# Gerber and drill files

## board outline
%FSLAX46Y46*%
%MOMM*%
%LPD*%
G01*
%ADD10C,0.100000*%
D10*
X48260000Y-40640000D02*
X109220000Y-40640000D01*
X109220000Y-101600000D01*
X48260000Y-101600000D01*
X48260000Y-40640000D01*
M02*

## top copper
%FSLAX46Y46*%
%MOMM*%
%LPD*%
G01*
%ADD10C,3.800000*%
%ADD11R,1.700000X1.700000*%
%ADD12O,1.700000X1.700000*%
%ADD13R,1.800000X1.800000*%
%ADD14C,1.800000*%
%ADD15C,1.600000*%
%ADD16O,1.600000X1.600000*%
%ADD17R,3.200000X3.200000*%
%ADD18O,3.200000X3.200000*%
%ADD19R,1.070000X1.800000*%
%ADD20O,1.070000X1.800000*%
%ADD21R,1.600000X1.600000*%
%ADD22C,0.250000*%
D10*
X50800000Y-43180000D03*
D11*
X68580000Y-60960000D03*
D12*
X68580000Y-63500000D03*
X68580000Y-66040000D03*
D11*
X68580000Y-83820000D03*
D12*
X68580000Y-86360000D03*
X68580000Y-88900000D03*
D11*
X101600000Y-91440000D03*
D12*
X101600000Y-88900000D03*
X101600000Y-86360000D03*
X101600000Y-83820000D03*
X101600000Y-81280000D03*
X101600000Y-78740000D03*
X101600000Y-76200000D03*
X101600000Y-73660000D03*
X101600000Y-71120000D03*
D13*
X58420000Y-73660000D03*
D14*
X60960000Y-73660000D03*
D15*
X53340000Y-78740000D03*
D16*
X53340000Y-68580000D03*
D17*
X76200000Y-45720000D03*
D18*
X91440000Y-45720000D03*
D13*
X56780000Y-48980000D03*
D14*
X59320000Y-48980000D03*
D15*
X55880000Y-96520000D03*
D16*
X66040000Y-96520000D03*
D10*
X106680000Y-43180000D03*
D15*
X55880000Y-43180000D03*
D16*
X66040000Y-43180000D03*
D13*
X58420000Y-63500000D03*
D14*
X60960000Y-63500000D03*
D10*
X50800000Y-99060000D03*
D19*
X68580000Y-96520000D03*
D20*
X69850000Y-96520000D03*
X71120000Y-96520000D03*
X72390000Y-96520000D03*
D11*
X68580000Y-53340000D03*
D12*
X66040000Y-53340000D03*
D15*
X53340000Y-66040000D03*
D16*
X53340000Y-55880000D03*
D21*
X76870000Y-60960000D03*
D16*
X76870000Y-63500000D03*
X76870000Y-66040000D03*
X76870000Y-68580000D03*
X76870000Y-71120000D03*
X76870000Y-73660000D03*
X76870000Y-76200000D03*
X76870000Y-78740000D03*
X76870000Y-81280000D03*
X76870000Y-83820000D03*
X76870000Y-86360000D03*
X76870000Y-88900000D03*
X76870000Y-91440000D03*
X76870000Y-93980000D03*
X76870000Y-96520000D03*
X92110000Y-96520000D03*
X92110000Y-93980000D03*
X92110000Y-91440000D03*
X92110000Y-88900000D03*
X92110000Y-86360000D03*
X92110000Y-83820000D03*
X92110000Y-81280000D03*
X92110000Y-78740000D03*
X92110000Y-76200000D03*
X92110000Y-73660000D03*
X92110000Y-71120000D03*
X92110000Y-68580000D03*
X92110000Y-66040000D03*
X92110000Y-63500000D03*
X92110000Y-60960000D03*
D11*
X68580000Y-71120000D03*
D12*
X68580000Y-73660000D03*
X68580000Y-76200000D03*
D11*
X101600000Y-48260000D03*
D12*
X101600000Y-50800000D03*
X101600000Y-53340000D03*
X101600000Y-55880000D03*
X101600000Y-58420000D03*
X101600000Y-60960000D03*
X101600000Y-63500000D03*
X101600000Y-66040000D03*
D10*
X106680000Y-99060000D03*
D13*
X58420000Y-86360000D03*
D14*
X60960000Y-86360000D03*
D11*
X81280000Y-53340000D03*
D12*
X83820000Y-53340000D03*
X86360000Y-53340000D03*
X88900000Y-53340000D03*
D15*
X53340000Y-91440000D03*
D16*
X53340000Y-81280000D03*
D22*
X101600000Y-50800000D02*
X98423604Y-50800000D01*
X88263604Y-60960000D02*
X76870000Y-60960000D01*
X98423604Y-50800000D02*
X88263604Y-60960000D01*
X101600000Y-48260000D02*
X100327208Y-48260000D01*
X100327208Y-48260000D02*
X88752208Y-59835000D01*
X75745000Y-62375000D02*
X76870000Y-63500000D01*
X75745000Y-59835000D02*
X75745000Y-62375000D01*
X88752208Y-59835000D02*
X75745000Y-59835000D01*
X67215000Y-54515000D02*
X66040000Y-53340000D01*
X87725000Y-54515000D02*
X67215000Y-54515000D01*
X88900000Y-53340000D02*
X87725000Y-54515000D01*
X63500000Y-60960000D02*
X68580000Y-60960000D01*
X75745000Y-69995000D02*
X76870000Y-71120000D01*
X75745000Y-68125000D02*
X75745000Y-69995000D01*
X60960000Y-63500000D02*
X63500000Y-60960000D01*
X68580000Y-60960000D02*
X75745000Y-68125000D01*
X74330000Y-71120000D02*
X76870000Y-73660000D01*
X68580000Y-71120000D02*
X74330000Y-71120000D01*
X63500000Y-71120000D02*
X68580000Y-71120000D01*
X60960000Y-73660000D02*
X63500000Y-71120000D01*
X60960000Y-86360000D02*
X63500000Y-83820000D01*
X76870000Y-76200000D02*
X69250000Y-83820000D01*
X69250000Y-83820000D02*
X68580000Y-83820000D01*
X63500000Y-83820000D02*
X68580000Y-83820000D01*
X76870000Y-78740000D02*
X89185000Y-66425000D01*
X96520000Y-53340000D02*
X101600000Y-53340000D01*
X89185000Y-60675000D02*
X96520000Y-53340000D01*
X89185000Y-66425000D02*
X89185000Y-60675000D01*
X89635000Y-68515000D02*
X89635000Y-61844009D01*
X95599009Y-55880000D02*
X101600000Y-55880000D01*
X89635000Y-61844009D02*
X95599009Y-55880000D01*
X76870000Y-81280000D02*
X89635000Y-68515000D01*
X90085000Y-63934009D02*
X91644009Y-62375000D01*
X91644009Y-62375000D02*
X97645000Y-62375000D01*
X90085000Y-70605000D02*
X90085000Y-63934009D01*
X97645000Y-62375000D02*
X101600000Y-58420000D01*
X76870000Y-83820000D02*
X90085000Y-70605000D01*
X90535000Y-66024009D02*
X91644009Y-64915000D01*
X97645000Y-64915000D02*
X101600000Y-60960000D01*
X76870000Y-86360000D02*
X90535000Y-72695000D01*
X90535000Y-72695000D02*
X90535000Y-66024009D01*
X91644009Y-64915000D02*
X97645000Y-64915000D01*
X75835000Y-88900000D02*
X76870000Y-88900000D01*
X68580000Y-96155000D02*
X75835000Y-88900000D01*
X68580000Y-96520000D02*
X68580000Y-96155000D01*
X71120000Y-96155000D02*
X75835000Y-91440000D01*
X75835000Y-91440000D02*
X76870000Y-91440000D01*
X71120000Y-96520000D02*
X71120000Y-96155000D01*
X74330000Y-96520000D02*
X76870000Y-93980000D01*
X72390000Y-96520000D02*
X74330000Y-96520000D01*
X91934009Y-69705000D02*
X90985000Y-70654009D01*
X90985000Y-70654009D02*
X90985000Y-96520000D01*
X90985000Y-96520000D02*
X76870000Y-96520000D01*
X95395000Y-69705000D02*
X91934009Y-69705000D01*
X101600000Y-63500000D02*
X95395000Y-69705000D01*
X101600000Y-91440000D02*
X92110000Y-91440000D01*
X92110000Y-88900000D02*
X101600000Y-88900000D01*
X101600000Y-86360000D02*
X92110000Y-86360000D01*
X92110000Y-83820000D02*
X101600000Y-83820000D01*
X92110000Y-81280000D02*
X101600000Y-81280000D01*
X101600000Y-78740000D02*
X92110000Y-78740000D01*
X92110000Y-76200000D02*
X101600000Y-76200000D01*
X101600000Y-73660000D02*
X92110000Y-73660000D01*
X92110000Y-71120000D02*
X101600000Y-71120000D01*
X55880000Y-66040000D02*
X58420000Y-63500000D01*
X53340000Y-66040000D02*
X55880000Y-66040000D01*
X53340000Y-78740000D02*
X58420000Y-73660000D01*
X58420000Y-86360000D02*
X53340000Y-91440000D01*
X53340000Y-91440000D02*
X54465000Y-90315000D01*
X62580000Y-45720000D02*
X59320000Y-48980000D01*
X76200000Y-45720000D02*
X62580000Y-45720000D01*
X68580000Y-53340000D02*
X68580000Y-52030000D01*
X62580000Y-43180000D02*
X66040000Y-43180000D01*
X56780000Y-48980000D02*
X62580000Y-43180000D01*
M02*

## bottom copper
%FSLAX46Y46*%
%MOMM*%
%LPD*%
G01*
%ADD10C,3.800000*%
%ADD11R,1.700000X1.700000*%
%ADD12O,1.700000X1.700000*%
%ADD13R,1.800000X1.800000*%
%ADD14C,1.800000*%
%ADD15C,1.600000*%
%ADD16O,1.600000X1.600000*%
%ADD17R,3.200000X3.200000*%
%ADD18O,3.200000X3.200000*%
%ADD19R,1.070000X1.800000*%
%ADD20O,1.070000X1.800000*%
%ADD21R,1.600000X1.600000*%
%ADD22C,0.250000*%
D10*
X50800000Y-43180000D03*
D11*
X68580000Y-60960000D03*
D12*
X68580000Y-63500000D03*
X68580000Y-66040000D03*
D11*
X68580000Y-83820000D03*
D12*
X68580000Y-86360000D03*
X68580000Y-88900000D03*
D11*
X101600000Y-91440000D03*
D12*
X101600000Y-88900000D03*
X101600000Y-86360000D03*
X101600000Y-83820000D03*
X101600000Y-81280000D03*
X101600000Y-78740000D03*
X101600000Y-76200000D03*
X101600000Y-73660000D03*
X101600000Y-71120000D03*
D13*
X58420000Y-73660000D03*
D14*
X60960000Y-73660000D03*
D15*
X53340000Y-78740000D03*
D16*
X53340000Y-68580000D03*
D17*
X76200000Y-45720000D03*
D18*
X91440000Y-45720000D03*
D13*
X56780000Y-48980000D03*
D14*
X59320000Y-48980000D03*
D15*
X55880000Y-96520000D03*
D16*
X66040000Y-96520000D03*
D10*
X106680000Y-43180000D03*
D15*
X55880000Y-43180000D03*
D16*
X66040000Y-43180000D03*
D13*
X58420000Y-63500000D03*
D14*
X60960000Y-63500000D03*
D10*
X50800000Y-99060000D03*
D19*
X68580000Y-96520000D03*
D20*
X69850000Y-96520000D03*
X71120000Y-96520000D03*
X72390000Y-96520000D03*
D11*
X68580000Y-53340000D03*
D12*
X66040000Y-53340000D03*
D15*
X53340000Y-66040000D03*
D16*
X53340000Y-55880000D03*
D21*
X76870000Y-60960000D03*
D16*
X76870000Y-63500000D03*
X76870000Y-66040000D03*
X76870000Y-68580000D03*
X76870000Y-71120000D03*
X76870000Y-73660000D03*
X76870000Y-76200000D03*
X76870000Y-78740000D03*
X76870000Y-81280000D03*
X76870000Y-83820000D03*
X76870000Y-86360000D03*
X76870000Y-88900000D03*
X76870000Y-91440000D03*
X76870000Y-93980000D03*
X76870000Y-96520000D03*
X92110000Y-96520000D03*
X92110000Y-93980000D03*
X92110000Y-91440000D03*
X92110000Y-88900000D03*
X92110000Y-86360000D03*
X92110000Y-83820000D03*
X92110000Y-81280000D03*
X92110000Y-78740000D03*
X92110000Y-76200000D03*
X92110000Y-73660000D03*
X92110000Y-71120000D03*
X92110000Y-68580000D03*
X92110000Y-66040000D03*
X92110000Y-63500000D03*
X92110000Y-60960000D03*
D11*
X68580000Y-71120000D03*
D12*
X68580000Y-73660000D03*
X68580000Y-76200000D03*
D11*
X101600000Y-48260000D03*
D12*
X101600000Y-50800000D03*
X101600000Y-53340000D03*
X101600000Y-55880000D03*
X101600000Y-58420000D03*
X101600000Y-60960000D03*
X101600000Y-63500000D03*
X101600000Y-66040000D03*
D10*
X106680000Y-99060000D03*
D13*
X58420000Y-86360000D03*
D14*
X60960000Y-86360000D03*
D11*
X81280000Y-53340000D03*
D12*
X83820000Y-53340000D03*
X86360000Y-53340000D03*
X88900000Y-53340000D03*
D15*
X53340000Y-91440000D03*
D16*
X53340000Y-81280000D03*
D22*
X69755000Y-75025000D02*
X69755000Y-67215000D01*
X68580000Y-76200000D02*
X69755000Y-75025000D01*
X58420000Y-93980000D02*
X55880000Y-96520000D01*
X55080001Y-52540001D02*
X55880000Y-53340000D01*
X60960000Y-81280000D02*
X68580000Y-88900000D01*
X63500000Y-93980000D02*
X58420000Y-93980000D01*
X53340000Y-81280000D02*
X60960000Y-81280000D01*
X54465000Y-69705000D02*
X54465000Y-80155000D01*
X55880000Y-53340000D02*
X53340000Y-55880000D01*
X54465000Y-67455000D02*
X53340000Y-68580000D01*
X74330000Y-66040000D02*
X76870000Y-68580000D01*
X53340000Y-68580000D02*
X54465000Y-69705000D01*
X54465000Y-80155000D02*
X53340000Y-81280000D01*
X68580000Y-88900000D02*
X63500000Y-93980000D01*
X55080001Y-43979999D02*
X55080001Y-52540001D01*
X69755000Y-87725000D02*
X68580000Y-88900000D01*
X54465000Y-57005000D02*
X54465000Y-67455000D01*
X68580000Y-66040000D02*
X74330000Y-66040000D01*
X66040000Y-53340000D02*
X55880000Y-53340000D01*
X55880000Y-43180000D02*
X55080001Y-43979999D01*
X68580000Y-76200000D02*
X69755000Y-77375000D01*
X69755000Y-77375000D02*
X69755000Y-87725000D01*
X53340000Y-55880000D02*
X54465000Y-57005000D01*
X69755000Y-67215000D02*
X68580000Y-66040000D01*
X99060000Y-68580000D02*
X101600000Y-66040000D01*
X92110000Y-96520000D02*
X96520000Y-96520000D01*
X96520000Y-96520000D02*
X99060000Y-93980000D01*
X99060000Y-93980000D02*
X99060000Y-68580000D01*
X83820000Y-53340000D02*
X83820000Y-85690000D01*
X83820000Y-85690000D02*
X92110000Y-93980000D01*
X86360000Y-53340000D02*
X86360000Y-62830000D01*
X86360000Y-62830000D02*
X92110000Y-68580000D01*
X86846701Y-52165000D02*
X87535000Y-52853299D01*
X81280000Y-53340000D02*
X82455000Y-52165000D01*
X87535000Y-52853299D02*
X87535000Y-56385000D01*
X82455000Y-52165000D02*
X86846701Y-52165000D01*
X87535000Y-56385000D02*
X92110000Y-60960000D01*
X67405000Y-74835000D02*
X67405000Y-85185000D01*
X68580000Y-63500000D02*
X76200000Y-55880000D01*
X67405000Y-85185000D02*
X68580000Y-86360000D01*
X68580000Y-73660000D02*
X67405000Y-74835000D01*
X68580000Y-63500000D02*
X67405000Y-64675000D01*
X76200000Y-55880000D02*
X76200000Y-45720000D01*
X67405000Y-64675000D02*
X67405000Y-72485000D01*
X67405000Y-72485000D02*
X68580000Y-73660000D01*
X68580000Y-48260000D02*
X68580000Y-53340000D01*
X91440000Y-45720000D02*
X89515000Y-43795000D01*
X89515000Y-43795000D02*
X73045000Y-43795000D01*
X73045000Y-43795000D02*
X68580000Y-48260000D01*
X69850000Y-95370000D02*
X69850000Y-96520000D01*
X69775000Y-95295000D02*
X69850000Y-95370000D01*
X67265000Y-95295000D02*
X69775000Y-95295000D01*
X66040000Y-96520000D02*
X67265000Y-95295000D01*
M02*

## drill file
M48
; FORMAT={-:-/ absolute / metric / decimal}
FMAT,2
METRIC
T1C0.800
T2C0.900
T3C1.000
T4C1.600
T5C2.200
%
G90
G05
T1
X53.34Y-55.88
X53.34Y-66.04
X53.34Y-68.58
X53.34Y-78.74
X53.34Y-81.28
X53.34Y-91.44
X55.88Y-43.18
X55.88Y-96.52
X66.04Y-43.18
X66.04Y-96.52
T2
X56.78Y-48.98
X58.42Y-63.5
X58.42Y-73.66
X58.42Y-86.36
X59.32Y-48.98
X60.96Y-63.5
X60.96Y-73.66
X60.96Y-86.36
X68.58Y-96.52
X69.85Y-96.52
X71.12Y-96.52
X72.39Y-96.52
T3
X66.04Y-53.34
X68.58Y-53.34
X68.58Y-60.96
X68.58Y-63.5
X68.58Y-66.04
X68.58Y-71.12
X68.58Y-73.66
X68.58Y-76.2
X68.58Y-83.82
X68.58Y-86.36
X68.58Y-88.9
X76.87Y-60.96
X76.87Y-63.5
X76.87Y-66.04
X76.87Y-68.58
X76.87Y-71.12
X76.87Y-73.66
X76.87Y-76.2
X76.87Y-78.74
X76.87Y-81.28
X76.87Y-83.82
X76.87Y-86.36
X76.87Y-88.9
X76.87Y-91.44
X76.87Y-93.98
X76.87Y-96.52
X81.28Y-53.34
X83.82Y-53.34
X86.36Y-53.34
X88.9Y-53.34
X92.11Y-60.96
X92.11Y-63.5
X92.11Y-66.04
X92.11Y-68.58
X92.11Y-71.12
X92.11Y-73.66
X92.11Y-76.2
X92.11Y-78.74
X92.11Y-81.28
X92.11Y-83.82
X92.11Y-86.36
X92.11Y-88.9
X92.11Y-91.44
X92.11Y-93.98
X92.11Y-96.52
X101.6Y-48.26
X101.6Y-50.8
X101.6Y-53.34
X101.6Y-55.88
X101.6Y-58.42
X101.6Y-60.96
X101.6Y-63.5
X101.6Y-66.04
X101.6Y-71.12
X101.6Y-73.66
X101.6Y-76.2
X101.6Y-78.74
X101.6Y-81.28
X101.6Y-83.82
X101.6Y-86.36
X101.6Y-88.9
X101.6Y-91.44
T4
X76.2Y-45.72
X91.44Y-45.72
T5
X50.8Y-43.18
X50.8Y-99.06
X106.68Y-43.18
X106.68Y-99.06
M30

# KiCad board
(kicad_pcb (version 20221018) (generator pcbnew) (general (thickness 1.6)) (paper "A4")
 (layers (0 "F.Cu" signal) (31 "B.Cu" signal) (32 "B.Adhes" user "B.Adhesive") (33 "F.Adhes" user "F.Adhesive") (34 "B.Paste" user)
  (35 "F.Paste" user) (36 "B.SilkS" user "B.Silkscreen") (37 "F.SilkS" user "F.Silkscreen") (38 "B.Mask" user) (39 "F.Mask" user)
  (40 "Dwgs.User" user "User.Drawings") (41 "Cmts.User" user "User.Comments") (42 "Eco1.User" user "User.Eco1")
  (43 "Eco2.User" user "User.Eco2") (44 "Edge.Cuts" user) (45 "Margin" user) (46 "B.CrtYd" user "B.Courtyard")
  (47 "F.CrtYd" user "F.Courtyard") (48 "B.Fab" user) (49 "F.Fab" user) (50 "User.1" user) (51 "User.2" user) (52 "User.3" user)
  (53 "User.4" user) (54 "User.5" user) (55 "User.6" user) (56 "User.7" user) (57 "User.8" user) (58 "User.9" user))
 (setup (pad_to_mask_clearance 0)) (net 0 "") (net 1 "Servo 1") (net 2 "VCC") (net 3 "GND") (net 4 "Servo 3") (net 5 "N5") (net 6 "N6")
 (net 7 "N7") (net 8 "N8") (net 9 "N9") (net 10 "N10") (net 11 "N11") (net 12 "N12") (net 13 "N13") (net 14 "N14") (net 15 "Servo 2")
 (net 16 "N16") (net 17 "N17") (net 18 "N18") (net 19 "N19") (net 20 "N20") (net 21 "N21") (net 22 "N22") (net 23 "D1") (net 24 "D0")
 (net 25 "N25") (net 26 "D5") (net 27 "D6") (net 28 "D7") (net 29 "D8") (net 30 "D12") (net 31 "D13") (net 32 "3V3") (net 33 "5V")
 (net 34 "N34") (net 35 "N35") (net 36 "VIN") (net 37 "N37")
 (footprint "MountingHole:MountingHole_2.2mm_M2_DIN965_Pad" (layer "F.Cu") (at 50.8 43.18)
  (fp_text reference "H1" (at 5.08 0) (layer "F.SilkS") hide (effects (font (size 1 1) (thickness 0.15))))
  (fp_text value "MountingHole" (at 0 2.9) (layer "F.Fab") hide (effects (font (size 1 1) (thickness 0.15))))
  (pad "1" thru_hole circle (at 0 0) (size 3.8 3.8) (drill 2.2) (layers "*.Cu" "*.Mask")))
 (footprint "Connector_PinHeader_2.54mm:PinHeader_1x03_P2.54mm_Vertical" (layer "F.Cu") (at 68.58 60.96)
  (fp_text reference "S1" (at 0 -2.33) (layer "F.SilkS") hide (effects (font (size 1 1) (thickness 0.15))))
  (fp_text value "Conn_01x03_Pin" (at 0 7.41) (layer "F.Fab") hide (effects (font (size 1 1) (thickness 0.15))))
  (pad "1" thru_hole rect (at 0 0) (size 1.7 1.7) (drill 1) (layers "*.Cu" "*.Mask") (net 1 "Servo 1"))
  (pad "2" thru_hole oval (at 0 2.54) (size 1.7 1.7) (drill 1) (layers "*.Cu" "*.Mask") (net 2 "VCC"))
  (pad "3" thru_hole oval (at 0 5.08) (size 1.7 1.7) (drill 1) (layers "*.Cu" "*.Mask") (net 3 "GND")))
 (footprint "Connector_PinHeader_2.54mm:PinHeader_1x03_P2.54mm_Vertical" (layer "F.Cu") (at 68.58 83.82)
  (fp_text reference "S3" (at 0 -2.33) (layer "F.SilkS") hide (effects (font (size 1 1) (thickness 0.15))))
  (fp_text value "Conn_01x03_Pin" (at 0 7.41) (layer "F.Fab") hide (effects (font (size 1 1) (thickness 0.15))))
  (pad "1" thru_hole rect (at 0 0) (size 1.7 1.7) (drill 1) (layers "*.Cu" "*.Mask") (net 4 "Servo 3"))
  (pad "2" thru_hole oval (at 0 2.54) (size 1.7 1.7) (drill 1) (layers "*.Cu" "*.Mask") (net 2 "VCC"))
  (pad "3" thru_hole oval (at 0 5.08) (size 1.7 1.7) (drill 1) (layers "*.Cu" "*.Mask") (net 3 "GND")))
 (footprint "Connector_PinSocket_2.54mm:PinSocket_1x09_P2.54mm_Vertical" (layer "F.Cu") (at 101.6 91.44 180)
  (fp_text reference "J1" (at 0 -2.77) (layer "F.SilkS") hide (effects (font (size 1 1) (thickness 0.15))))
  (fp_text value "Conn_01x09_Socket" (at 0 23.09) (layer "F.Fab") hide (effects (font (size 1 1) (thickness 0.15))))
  (pad "1" thru_hole rect (at 0 0 180) (size 1.7 1.7) (drill 1) (layers "*.Cu" "*.Mask") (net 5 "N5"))
  (pad "2" thru_hole oval (at 0 2.54 180) (size 1.7 1.7) (drill 1) (layers "*.Cu" "*.Mask") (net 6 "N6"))
  (pad "3" thru_hole oval (at 0 5.08 180) (size 1.7 1.7) (drill 1) (layers "*.Cu" "*.Mask") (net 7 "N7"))
  (pad "4" thru_hole oval (at 0 7.62 180) (size 1.7 1.7) (drill 1) (layers "*.Cu" "*.Mask") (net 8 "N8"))
  (pad "5" thru_hole oval (at 0 10.16 180) (size 1.7 1.7) (drill 1) (layers "*.Cu" "*.Mask") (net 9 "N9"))
  (pad "6" thru_hole oval (at 0 12.7 180) (size 1.7 1.7) (drill 1) (layers "*.Cu" "*.Mask") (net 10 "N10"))
  (pad "7" thru_hole oval (at 0 15.24 180) (size 1.7 1.7) (drill 1) (layers "*.Cu" "*.Mask") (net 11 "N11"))
  (pad "8" thru_hole oval (at 0 17.78 180) (size 1.7 1.7) (drill 1) (layers "*.Cu" "*.Mask") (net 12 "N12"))
  (pad "9" thru_hole oval (at 0 20.32 180) (size 1.7 1.7) (drill 1) (layers "*.Cu" "*.Mask") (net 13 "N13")))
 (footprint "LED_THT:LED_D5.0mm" (layer "F.Cu") (at 58.42 73.66)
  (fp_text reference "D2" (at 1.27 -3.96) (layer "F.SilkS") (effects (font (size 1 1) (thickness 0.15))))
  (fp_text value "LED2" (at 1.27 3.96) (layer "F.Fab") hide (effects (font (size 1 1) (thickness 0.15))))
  (pad "1" thru_hole rect (at 0 0) (size 1.8 1.8) (drill 0.9) (layers "*.Cu" "*.Mask") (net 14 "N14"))
  (pad "2" thru_hole circle (at 2.54 0) (size 1.8 1.8) (drill 0.9) (layers "*.Cu" "*.Mask") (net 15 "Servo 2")))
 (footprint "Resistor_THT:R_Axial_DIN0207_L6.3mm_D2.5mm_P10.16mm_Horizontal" (layer "F.Cu") (at 53.34 78.74 90)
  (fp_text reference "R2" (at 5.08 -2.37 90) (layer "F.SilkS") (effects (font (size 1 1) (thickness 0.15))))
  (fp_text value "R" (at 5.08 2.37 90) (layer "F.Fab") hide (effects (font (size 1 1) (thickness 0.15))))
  (pad "1" thru_hole circle (at 0 0 90) (size 1.6 1.6) (drill 0.8) (layers "*.Cu" "*.Mask") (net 14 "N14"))
  (pad "2" thru_hole oval (at 10.16 0 90) (size 1.6 1.6) (drill 0.8) (layers "*.Cu" "*.Mask") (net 3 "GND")))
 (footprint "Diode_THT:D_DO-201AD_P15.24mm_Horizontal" (layer "F.Cu") (at 76.2 45.72)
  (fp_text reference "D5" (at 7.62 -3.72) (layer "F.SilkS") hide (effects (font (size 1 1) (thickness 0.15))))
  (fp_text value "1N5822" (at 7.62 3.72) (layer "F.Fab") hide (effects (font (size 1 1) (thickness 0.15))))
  (pad "1" thru_hole rect (at 0 0) (size 3.2 3.2) (drill 1.6) (layers "*.Cu" "*.Mask") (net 2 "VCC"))
  (pad "2" thru_hole oval (at 15.24 0) (size 3.2 3.2) (drill 1.6) (layers "*.Cu" "*.Mask") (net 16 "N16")))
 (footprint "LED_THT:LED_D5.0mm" (layer "F.Cu") (at 56.78 48.98)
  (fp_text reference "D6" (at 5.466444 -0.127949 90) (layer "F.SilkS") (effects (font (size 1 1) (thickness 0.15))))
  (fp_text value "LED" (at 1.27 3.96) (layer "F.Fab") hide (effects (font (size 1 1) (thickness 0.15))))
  (pad "1" thru_hole rect (at 0 0) (size 1.8 1.8) (drill 0.9) (layers "*.Cu" "*.Mask") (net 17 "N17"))
  (pad "2" thru_hole circle (at 2.54 0) (size 1.8 1.8) (drill 0.9) (layers "*.Cu" "*.Mask") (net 2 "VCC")))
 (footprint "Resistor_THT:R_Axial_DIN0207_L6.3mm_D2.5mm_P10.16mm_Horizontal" (layer "F.Cu") (at 55.88 96.52)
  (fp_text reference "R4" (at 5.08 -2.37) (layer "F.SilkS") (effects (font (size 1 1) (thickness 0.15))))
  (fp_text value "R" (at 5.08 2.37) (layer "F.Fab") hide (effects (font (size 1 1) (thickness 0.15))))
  (pad "1" thru_hole circle (at 0 0) (size 1.6 1.6) (drill 0.8) (layers "*.Cu" "*.Mask") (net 3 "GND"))
  (pad "2" thru_hole oval (at 10.16 0) (size 1.6 1.6) (drill 0.8) (layers "*.Cu" "*.Mask") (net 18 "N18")))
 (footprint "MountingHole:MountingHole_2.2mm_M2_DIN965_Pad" (layer "F.Cu") (at 106.68 43.18)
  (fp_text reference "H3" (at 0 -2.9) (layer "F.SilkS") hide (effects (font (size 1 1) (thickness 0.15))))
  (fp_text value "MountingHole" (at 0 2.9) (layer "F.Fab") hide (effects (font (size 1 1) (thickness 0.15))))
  (pad "1" thru_hole circle (at 0 0) (size 3.8 3.8) (drill 2.2) (layers "*.Cu" "*.Mask")))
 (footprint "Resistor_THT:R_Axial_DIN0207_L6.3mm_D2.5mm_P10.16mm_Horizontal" (layer "F.Cu") (at 55.88 43.18)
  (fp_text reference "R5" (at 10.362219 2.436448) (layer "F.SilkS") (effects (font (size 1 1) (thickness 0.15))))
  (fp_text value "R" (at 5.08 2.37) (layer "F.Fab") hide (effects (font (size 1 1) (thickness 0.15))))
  (pad "1" thru_hole circle (at 0 0) (size 1.6 1.6) (drill 0.8) (layers "*.Cu" "*.Mask") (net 3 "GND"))
  (pad "2" thru_hole oval (at 10.16 0) (size 1.6 1.6) (drill 0.8) (layers "*.Cu" "*.Mask") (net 17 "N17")))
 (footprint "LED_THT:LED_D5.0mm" (layer "F.Cu") (at 58.42 63.5)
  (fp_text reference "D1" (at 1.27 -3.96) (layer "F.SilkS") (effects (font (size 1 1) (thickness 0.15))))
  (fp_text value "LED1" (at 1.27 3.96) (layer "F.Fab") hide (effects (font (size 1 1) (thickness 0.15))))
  (pad "1" thru_hole rect (at 0 0) (size 1.8 1.8) (drill 0.9) (layers "*.Cu" "*.Mask") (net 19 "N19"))
  (pad "2" thru_hole circle (at 2.54 0) (size 1.8 1.8) (drill 0.9) (layers "*.Cu" "*.Mask") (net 1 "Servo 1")))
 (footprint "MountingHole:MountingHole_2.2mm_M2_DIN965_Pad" (layer "F.Cu") (at 50.8 99.06)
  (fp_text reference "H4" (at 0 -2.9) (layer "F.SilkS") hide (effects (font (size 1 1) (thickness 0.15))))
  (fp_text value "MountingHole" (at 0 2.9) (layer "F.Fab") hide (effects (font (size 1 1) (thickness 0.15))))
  (pad "1" thru_hole circle (at 0 0) (size 3.8 3.8) (drill 2.2) (layers "*.Cu" "*.Mask")))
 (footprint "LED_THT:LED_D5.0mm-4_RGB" (layer "F.Cu") (at 68.58 96.52)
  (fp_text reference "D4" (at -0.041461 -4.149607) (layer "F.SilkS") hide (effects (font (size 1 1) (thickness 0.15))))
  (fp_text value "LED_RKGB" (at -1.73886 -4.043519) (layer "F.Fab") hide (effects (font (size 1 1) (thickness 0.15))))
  (pad "1" thru_hole rect (at 0 0) (size 1.07 1.8) (drill 0.9) (layers "*.Cu" "*.Mask") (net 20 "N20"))
  (pad "2" thru_hole oval (at 1.27 0) (size 1.07 1.8) (drill 0.9) (layers "*.Cu" "*.Mask") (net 18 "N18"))
  (pad "3" thru_hole oval (at 2.54 0) (size 1.07 1.8) (drill 0.9) (layers "*.Cu" "*.Mask") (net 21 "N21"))
  (pad "4" thru_hole oval (at 3.81 0) (size 1.07 1.8) (drill 0.9) (layers "*.Cu" "*.Mask") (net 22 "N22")))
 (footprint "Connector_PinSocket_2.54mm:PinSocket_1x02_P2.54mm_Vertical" (layer "F.Cu") (at 68.58 53.34 -90)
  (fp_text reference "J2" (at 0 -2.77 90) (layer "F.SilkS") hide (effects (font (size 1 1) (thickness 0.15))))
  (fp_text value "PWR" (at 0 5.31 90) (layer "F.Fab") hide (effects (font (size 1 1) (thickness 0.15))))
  (pad "1" thru_hole rect (at 0 0 270) (size 1.7 1.7) (drill 1) (layers "*.Cu" "*.Mask") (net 16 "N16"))
  (pad "2" thru_hole oval (at 0 2.54 270) (size 1.7 1.7) (drill 1) (layers "*.Cu" "*.Mask") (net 3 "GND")))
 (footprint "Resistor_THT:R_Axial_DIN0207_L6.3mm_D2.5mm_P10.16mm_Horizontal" (layer "F.Cu") (at 53.34 66.04 90)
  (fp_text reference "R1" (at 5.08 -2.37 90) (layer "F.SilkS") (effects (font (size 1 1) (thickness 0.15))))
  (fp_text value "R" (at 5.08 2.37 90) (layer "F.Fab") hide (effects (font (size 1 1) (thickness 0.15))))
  (pad "1" thru_hole circle (at 0 0 90) (size 1.6 1.6) (drill 0.8) (layers "*.Cu" "*.Mask") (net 19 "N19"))
  (pad "2" thru_hole oval (at 10.16 0 90) (size 1.6 1.6) (drill 0.8) (layers "*.Cu" "*.Mask") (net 3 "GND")))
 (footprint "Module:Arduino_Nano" (layer "F.Cu") (at 76.87 60.96)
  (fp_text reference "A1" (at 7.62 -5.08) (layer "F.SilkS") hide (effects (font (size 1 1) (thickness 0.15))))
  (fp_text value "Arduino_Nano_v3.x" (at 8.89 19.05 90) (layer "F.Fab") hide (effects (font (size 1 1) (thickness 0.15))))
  (pad "1" thru_hole rect (at 0 0) (size 1.6 1.6) (drill 1) (layers "*.Cu" "*.Mask") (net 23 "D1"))
  (pad "2" thru_hole oval (at 0 2.54) (size 1.6 1.6) (drill 1) (layers "*.Cu" "*.Mask") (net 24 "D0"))
  (pad "3" thru_hole oval (at 0 5.08) (size 1.6 1.6) (drill 1) (layers "*.Cu" "*.Mask") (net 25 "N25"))
  (pad "4" thru_hole oval (at 0 7.62) (size 1.6 1.6) (drill 1) (layers "*.Cu" "*.Mask") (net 3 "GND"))
  (pad "5" thru_hole oval (at 0 10.16) (size 1.6 1.6) (drill 1) (layers "*.Cu" "*.Mask") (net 1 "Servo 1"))
  (pad "6" thru_hole oval (at 0 12.7) (size 1.6 1.6) (drill 1) (layers "*.Cu" "*.Mask") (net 15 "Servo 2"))
  (pad "7" thru_hole oval (at 0 15.24) (size 1.6 1.6) (drill 1) (layers "*.Cu" "*.Mask") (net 4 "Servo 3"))
  (pad "8" thru_hole oval (at 0 17.78) (size 1.6 1.6) (drill 1) (layers "*.Cu" "*.Mask") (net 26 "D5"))
  (pad "9" thru_hole oval (at 0 20.32) (size 1.6 1.6) (drill 1) (layers "*.Cu" "*.Mask") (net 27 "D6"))
  (pad "10" thru_hole oval (at 0 22.86) (size 1.6 1.6) (drill 1) (layers "*.Cu" "*.Mask") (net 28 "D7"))
  (pad "11" thru_hole oval (at 0 25.4) (size 1.6 1.6) (drill 1) (layers "*.Cu" "*.Mask") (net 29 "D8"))
  (pad "12" thru_hole oval (at 0 27.94) (size 1.6 1.6) (drill 1) (layers "*.Cu" "*.Mask") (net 20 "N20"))
  (pad "13" thru_hole oval (at 0 30.48) (size 1.6 1.6) (drill 1) (layers "*.Cu" "*.Mask") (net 21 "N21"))
  (pad "14" thru_hole oval (at 0 33.02) (size 1.6 1.6) (drill 1) (layers "*.Cu" "*.Mask") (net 22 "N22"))
  (pad "15" thru_hole oval (at 0 35.56) (size 1.6 1.6) (drill 1) (layers "*.Cu" "*.Mask") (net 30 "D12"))
  (pad "16" thru_hole oval (at 15.24 35.56) (size 1.6 1.6) (drill 1) (layers "*.Cu" "*.Mask") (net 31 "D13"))
  (pad "17" thru_hole oval (at 15.24 33.02) (size 1.6 1.6) (drill 1) (layers "*.Cu" "*.Mask") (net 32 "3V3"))
  (pad "18" thru_hole oval (at 15.24 30.48) (size 1.6 1.6) (drill 1) (layers "*.Cu" "*.Mask") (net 5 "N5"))
  (pad "19" thru_hole oval (at 15.24 27.94) (size 1.6 1.6) (drill 1) (layers "*.Cu" "*.Mask") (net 6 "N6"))
  (pad "20" thru_hole oval (at 15.24 25.4) (size 1.6 1.6) (drill 1) (layers "*.Cu" "*.Mask") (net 7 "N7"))
  (pad "21" thru_hole oval (at 15.24 22.86) (size 1.6 1.6) (drill 1) (layers "*.Cu" "*.Mask") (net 8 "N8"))
  (pad "22" thru_hole oval (at 15.24 20.32) (size 1.6 1.6) (drill 1) (layers "*.Cu" "*.Mask") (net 9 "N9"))
  (pad "23" thru_hole oval (at 15.24 17.78) (size 1.6 1.6) (drill 1) (layers "*.Cu" "*.Mask") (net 10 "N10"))
  (pad "24" thru_hole oval (at 15.24 15.24) (size 1.6 1.6) (drill 1) (layers "*.Cu" "*.Mask") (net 11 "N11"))
  (pad "25" thru_hole oval (at 15.24 12.7) (size 1.6 1.6) (drill 1) (layers "*.Cu" "*.Mask") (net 12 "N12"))
  (pad "26" thru_hole oval (at 15.24 10.16) (size 1.6 1.6) (drill 1) (layers "*.Cu" "*.Mask") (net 13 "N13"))
  (pad "27" thru_hole oval (at 15.24 7.62) (size 1.6 1.6) (drill 1) (layers "*.Cu" "*.Mask") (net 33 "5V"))
  (pad "28" thru_hole oval (at 15.24 5.08) (size 1.6 1.6) (drill 1) (layers "*.Cu" "*.Mask") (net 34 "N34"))
  (pad "29" thru_hole oval (at 15.24 2.54) (size 1.6 1.6) (drill 1) (layers "*.Cu" "*.Mask") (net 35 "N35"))
  (pad "30" thru_hole oval (at 15.24 0) (size 1.6 1.6) (drill 1) (layers "*.Cu" "*.Mask") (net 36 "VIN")))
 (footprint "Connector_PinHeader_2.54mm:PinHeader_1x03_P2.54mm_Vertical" (layer "F.Cu") (at 68.58 71.12)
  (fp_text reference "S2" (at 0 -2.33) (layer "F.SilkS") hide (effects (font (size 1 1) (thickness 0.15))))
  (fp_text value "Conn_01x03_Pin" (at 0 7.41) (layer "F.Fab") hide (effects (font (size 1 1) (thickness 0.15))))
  (pad "1" thru_hole rect (at 0 0) (size 1.7 1.7) (drill 1) (layers "*.Cu" "*.Mask") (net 15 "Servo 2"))
  (pad "2" thru_hole oval (at 0 2.54) (size 1.7 1.7) (drill 1) (layers "*.Cu" "*.Mask") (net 2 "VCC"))
  (pad "3" thru_hole oval (at 0 5.08) (size 1.7 1.7) (drill 1) (layers "*.Cu" "*.Mask") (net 3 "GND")))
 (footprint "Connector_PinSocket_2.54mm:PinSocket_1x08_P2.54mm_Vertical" (layer "F.Cu") (at 101.6 48.26)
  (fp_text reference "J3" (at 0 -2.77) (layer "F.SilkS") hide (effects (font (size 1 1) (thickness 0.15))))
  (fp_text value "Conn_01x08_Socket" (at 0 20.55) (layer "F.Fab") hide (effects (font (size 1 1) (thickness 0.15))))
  (pad "1" thru_hole rect (at 0 0) (size 1.7 1.7) (drill 1) (layers "*.Cu" "*.Mask") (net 24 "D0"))
  (pad "2" thru_hole oval (at 0 2.54) (size 1.7 1.7) (drill 1) (layers "*.Cu" "*.Mask") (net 23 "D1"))
  (pad "3" thru_hole oval (at 0 5.08) (size 1.7 1.7) (drill 1) (layers "*.Cu" "*.Mask") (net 26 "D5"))
  (pad "4" thru_hole oval (at 0 7.62) (size 1.7 1.7) (drill 1) (layers "*.Cu" "*.Mask") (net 27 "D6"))
  (pad "5" thru_hole oval (at 0 10.16) (size 1.7 1.7) (drill 1) (layers "*.Cu" "*.Mask") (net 28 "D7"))
  (pad "6" thru_hole oval (at 0 12.7) (size 1.7 1.7) (drill 1) (layers "*.Cu" "*.Mask") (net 29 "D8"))
  (pad "7" thru_hole oval (at 0 15.24) (size 1.7 1.7) (drill 1) (layers "*.Cu" "*.Mask") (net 30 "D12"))
  (pad "8" thru_hole oval (at 0 17.78) (size 1.7 1.7) (drill 1) (layers "*.Cu" "*.Mask") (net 31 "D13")))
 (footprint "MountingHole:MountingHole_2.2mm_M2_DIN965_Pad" (layer "F.Cu") (at 106.68 99.06)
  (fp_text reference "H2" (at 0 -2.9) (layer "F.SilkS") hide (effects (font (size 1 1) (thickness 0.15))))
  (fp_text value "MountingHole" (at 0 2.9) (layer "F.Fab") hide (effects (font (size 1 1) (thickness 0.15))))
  (pad "1" thru_hole circle (at 0 0) (size 3.8 3.8) (drill 2.2) (layers "*.Cu" "*.Mask")))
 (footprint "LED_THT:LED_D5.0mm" (layer "F.Cu") (at 58.42 86.36)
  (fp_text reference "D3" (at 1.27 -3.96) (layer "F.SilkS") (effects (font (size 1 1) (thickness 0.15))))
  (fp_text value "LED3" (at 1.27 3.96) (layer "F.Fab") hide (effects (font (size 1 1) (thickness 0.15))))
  (pad "1" thru_hole rect (at 0 0) (size 1.8 1.8) (drill 0.9) (layers "*.Cu" "*.Mask") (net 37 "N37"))
  (pad "2" thru_hole circle (at 2.54 0) (size 1.8 1.8) (drill 0.9) (layers "*.Cu" "*.Mask") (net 4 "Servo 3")))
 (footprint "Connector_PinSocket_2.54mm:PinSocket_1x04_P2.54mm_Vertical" (layer "F.Cu") (at 81.28 53.34 90)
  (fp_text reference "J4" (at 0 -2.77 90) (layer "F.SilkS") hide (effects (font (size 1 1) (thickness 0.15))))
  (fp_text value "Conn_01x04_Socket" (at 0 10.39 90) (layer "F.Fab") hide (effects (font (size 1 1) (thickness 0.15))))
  (pad "1" thru_hole rect (at 0 0 90) (size 1.7 1.7) (drill 1) (layers "*.Cu" "*.Mask") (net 36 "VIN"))
  (pad "2" thru_hole oval (at 0 2.54 90) (size 1.7 1.7) (drill 1) (layers "*.Cu" "*.Mask") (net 32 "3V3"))
  (pad "3" thru_hole oval (at 0 5.08 90) (size 1.7 1.7) (drill 1) (layers "*.Cu" "*.Mask") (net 33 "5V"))
  (pad "4" thru_hole oval (at 0 7.62 90) (size 1.7 1.7) (drill 1) (layers "*.Cu" "*.Mask") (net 3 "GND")))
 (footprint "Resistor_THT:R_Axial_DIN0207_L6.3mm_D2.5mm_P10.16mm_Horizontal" (layer "F.Cu") (at 53.34 91.44 90)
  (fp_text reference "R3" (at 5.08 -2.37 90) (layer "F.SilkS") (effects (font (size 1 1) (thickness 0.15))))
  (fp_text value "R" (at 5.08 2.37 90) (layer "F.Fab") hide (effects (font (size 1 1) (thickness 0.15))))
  (pad "1" thru_hole circle (at 0 0 90) (size 1.6 1.6) (drill 0.8) (layers "*.Cu" "*.Mask") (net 37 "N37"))
  (pad "2" thru_hole oval (at 10.16 0 90) (size 1.6 1.6) (drill 0.8) (layers "*.Cu" "*.Mask") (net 3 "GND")))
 (gr_rect (start 48.26 40.64) (end 109.22 101.6) (stroke (width 0.1) (type default)) (fill none) (layer "Edge.Cuts"))
 (segment (start 101.6 50.8) (end 98.423604 50.8) (width 0.25) (layer "F.Cu") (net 23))
 (segment (start 88.263604 60.96) (end 76.87 60.96) (width 0.25) (layer "F.Cu") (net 23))
 (segment (start 98.423604 50.8) (end 88.263604 60.96) (width 0.25) (layer "F.Cu") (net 23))
 (segment (start 101.6 48.26) (end 100.327208 48.26) (width 0.25) (layer "F.Cu") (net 24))
 (segment (start 100.327208 48.26) (end 88.752208 59.835) (width 0.25) (layer "F.Cu") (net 24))
 (segment (start 75.745 62.375) (end 76.87 63.5) (width 0.25) (layer "F.Cu") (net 24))
 (segment (start 75.745 59.835) (end 75.745 62.375) (width 0.25) (layer "F.Cu") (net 24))
 (segment (start 88.752208 59.835) (end 75.745 59.835) (width 0.25) (layer "F.Cu") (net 24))
 (segment (start 67.215 54.515) (end 66.04 53.34) (width 0.25) (layer "F.Cu") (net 3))
 (segment (start 87.725 54.515) (end 67.215 54.515) (width 0.25) (layer "F.Cu") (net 3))
 (segment (start 88.9 53.34) (end 87.725 54.515) (width 0.25) (layer "F.Cu") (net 3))
 (segment (start 69.755 75.025) (end 69.755 67.215) (width 0.25) (layer "B.Cu") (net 3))
 (segment (start 68.58 76.2) (end 69.755 75.025) (width 0.25) (layer "B.Cu") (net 3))
 (segment (start 58.42 93.98) (end 55.88 96.52) (width 0.25) (layer "B.Cu") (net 3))
 (segment (start 55.080001 52.540001) (end 55.88 53.34) (width 0.25) (layer "B.Cu") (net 3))
 (segment (start 60.96 81.28) (end 68.58 88.9) (width 0.25) (layer "B.Cu") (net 3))
 (segment (start 63.5 93.98) (end 58.42 93.98) (width 0.25) (layer "B.Cu") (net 3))
 (segment (start 53.34 81.28) (end 60.96 81.28) (width 0.25) (layer "B.Cu") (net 3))
 (segment (start 54.465 69.705) (end 54.465 80.155) (width 0.25) (layer "B.Cu") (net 3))
 (segment (start 55.88 53.34) (end 53.34 55.88) (width 0.25) (layer "B.Cu") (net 3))
 (segment (start 54.465 67.455) (end 53.34 68.58) (width 0.25) (layer "B.Cu") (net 3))
 (segment (start 74.33 66.04) (end 76.87 68.58) (width 0.25) (layer "B.Cu") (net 3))
 (segment (start 53.34 68.58) (end 54.465 69.705) (width 0.25) (layer "B.Cu") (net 3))
 (segment (start 54.465 80.155) (end 53.34 81.28) (width 0.25) (layer "B.Cu") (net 3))
 (segment (start 68.58 88.9) (end 63.5 93.98) (width 0.25) (layer "B.Cu") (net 3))
 (segment (start 55.080001 43.979999) (end 55.080001 52.540001) (width 0.25) (layer "B.Cu") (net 3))
 (segment (start 69.755 87.725) (end 68.58 88.9) (width 0.25) (layer "B.Cu") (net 3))
 (segment (start 54.465 57.005) (end 54.465 67.455) (width 0.25) (layer "B.Cu") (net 3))
 (segment (start 68.58 66.04) (end 74.33 66.04) (width 0.25) (layer "B.Cu") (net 3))
 (segment (start 66.04 53.34) (end 55.88 53.34) (width 0.25) (layer "B.Cu") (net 3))
 (segment (start 55.88 43.18) (end 55.080001 43.979999) (width 0.25) (layer "B.Cu") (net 3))
 (segment (start 68.58 76.2) (end 69.755 77.375) (width 0.25) (layer "B.Cu") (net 3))
 (segment (start 69.755 77.375) (end 69.755 87.725) (width 0.25) (layer "B.Cu") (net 3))
 (segment (start 53.34 55.88) (end 54.465 57.005) (width 0.25) (layer "B.Cu") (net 3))
 (segment (start 69.755 67.215) (end 68.58 66.04) (width 0.25) (layer "B.Cu") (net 3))
 (segment (start 63.5 60.96) (end 68.58 60.96) (width 0.25) (layer "F.Cu") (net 1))
 (segment (start 75.745 69.995) (end 76.87 71.12) (width 0.25) (layer "F.Cu") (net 1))
 (segment (start 75.745 68.125) (end 75.745 69.995) (width 0.25) (layer "F.Cu") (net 1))
 (segment (start 60.96 63.5) (end 63.5 60.96) (width 0.25) (layer "F.Cu") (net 1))
 (segment (start 68.58 60.96) (end 75.745 68.125) (width 0.25) (layer "F.Cu") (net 1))
 (segment (start 74.33 71.12) (end 76.87 73.66) (width 0.25) (layer "F.Cu") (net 15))
 (segment (start 68.58 71.12) (end 74.33 71.12) (width 0.25) (layer "F.Cu") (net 15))
 (segment (start 63.5 71.12) (end 68.58 71.12) (width 0.25) (layer "F.Cu") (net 15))
 (segment (start 60.96 73.66) (end 63.5 71.12) (width 0.25) (layer "F.Cu") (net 15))
 (segment (start 60.96 86.36) (end 63.5 83.82) (width 0.25) (layer "F.Cu") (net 4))
 (segment (start 76.87 76.2) (end 69.25 83.82) (width 0.25) (layer "F.Cu") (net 4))
 (segment (start 69.25 83.82) (end 68.58 83.82) (width 0.25) (layer "F.Cu") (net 4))
 (segment (start 63.5 83.82) (end 68.58 83.82) (width 0.25) (layer "F.Cu") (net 4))
 (segment (start 76.87 78.74) (end 89.185 66.425) (width 0.25) (layer "F.Cu") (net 26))
 (segment (start 96.52 53.34) (end 101.6 53.34) (width 0.25) (layer "F.Cu") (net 26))
 (segment (start 89.185 60.675) (end 96.52 53.34) (width 0.25) (layer "F.Cu") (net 26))
 (segment (start 89.185 66.425) (end 89.185 60.675) (width 0.25) (layer "F.Cu") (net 26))
 (segment (start 89.635 68.515) (end 89.635 61.844009) (width 0.25) (layer "F.Cu") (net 27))
 (segment (start 95.599009 55.88) (end 101.6 55.88) (width 0.25) (layer "F.Cu") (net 27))
 (segment (start 89.635 61.844009) (end 95.599009 55.88) (width 0.25) (layer "F.Cu") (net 27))
 (segment (start 76.87 81.28) (end 89.635 68.515) (width 0.25) (layer "F.Cu") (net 27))
 (segment (start 90.085 63.934009) (end 91.644009 62.375) (width 0.25) (layer "F.Cu") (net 28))
 (segment (start 91.644009 62.375) (end 97.645 62.375) (width 0.25) (layer "F.Cu") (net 28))
 (segment (start 90.085 70.605) (end 90.085 63.934009) (width 0.25) (layer "F.Cu") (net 28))
 (segment (start 97.645 62.375) (end 101.6 58.42) (width 0.25) (layer "F.Cu") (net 28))
 (segment (start 76.87 83.82) (end 90.085 70.605) (width 0.25) (layer "F.Cu") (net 28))
 (segment (start 90.535 66.024009) (end 91.644009 64.915) (width 0.25) (layer "F.Cu") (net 29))
 (segment (start 97.645 64.915) (end 101.6 60.96) (width 0.25) (layer "F.Cu") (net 29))
 (segment (start 76.87 86.36) (end 90.535 72.695) (width 0.25) (layer "F.Cu") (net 29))
 (segment (start 90.535 72.695) (end 90.535 66.024009) (width 0.25) (layer "F.Cu") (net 29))
 (segment (start 91.644009 64.915) (end 97.645 64.915) (width 0.25) (layer "F.Cu") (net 29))
 (segment (start 75.835 88.9) (end 76.87 88.9) (width 0.25) (layer "F.Cu") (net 20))
 (segment (start 68.58 96.155) (end 75.835 88.9) (width 0.25) (layer "F.Cu") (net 20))
 (segment (start 68.58 96.52) (end 68.58 96.155) (width 0.25) (layer "F.Cu") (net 20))
 (segment (start 71.12 96.155) (end 75.835 91.44) (width 0.25) (layer "F.Cu") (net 21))
 (segment (start 75.835 91.44) (end 76.87 91.44) (width 0.25) (layer "F.Cu") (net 21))
 (segment (start 71.12 96.52) (end 71.12 96.155) (width 0.25) (layer "F.Cu") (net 21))
 (segment (start 74.33 96.52) (end 76.87 93.98) (width 0.25) (layer "F.Cu") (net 22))
 (segment (start 72.39 96.52) (end 74.33 96.52) (width 0.25) (layer "F.Cu") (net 22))
 (segment (start 91.934009 69.705) (end 90.985 70.654009) (width 0.25) (layer "F.Cu") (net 30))
 (segment (start 90.985 70.654009) (end 90.985 96.52) (width 0.25) (layer "F.Cu") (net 30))
 (segment (start 90.985 96.52) (end 76.87 96.52) (width 0.25) (layer "F.Cu") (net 30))
 (segment (start 95.395 69.705) (end 91.934009 69.705) (width 0.25) (layer "F.Cu") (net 30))
 (segment (start 101.6 63.5) (end 95.395 69.705) (width 0.25) (layer "F.Cu") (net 30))
 (segment (start 99.06 68.58) (end 101.6 66.04) (width 0.25) (layer "B.Cu") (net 31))
 (segment (start 92.11 96.52) (end 96.52 96.52) (width 0.25) (layer "B.Cu") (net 31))
 (segment (start 96.52 96.52) (end 99.06 93.98) (width 0.25) (layer "B.Cu") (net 31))
 (segment (start 99.06 93.98) (end 99.06 68.58) (width 0.25) (layer "B.Cu") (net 31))
 (segment (start 83.82 53.34) (end 83.82 85.69) (width 0.25) (layer "B.Cu") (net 32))
 (segment (start 83.82 85.69) (end 92.11 93.98) (width 0.25) (layer "B.Cu") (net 32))
 (segment (start 101.6 91.44) (end 92.11 91.44) (width 0.25) (layer "F.Cu") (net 5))
 (segment (start 92.11 88.9) (end 101.6 88.9) (width 0.25) (layer "F.Cu") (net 6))
 (segment (start 101.6 86.36) (end 92.11 86.36) (width 0.25) (layer "F.Cu") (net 7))
 (segment (start 92.11 83.82) (end 101.6 83.82) (width 0.25) (layer "F.Cu") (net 8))
 (segment (start 92.11 81.28) (end 101.6 81.28) (width 0.25) (layer "F.Cu") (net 9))
 (segment (start 101.6 78.74) (end 92.11 78.74) (width 0.25) (layer "F.Cu") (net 10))
 (segment (start 92.11 76.2) (end 101.6 76.2) (width 0.25) (layer "F.Cu") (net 11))
 (segment (start 101.6 73.66) (end 92.11 73.66) (width 0.25) (layer "F.Cu") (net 12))
 (segment (start 92.11 71.12) (end 101.6 71.12) (width 0.25) (layer "F.Cu") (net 13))
 (segment (start 86.36 53.34) (end 86.36 62.83) (width 0.25) (layer "B.Cu") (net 33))
 (segment (start 86.36 62.83) (end 92.11 68.58) (width 0.25) (layer "B.Cu") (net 33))
 (segment (start 86.846701 52.165) (end 87.535 52.853299) (width 0.25) (layer "B.Cu") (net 36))
 (segment (start 81.28 53.34) (end 82.455 52.165) (width 0.25) (layer "B.Cu") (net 36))
 (segment (start 87.535 52.853299) (end 87.535 56.385) (width 0.25) (layer "B.Cu") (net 36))
 (segment (start 82.455 52.165) (end 86.846701 52.165) (width 0.25) (layer "B.Cu") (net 36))
 (segment (start 87.535 56.385) (end 92.11 60.96) (width 0.25) (layer "B.Cu") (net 36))
 (segment (start 55.88 66.04) (end 58.42 63.5) (width 0.25) (layer "F.Cu") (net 19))
 (segment (start 53.34 66.04) (end 55.88 66.04) (width 0.25) (layer "F.Cu") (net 19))
 (segment (start 53.34 78.74) (end 58.42 73.66) (width 0.25) (layer "F.Cu") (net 14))
 (segment (start 58.42 86.36) (end 53.34 91.44) (width 0.25) (layer "F.Cu") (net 37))
 (segment (start 53.34 91.44) (end 54.465 90.315) (width 0.25) (layer "F.Cu") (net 37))
 (segment (start 62.58 45.72) (end 59.32 48.98) (width 0.25) (layer "F.Cu") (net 2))
 (segment (start 76.2 45.72) (end 62.58 45.72) (width 0.25) (layer "F.Cu") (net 2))
 (segment (start 67.405 74.835) (end 67.405 85.185) (width 0.25) (layer "B.Cu") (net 2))
 (segment (start 68.58 63.5) (end 76.2 55.88) (width 0.25) (layer "B.Cu") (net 2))
 (segment (start 67.405 85.185) (end 68.58 86.36) (width 0.25) (layer "B.Cu") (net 2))
 (segment (start 68.58 73.66) (end 67.405 74.835) (width 0.25) (layer "B.Cu") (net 2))
 (segment (start 68.58 63.5) (end 67.405 64.675) (width 0.25) (layer "B.Cu") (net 2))
 (segment (start 76.2 55.88) (end 76.2 45.72) (width 0.25) (layer "B.Cu") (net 2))
 (segment (start 67.405 64.675) (end 67.405 72.485) (width 0.25) (layer "B.Cu") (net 2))
 (segment (start 67.405 72.485) (end 68.58 73.66) (width 0.25) (layer "B.Cu") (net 2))
 (segment (start 68.58 53.34) (end 68.58 52.03) (width 0.25) (layer "F.Cu") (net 16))
 (segment (start 68.58 48.26) (end 68.58 53.34) (width 0.25) (layer "B.Cu") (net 16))
 (segment (start 91.44 45.72) (end 89.515 43.795) (width 0.25) (layer "B.Cu") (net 16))
 (segment (start 89.515 43.795) (end 73.045 43.795) (width 0.25) (layer "B.Cu") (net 16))
 (segment (start 73.045 43.795) (end 68.58 48.26) (width 0.25) (layer "B.Cu") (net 16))
 (segment (start 69.85 95.37) (end 69.85 96.52) (width 0.25) (layer "B.Cu") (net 18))
 (segment (start 69.775 95.295) (end 69.85 95.37) (width 0.25) (layer "B.Cu") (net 18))
 (segment (start 67.265 95.295) (end 69.775 95.295) (width 0.25) (layer "B.Cu") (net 18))
 (segment (start 66.04 96.52) (end 67.265 95.295) (width 0.25) (layer "B.Cu") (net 18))
 (segment (start 62.58 43.18) (end 66.04 43.18) (width 0.25) (layer "F.Cu") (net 17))
 (segment (start 56.78 48.98) (end 62.58 43.18) (width 0.25) (layer "F.Cu") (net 17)))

